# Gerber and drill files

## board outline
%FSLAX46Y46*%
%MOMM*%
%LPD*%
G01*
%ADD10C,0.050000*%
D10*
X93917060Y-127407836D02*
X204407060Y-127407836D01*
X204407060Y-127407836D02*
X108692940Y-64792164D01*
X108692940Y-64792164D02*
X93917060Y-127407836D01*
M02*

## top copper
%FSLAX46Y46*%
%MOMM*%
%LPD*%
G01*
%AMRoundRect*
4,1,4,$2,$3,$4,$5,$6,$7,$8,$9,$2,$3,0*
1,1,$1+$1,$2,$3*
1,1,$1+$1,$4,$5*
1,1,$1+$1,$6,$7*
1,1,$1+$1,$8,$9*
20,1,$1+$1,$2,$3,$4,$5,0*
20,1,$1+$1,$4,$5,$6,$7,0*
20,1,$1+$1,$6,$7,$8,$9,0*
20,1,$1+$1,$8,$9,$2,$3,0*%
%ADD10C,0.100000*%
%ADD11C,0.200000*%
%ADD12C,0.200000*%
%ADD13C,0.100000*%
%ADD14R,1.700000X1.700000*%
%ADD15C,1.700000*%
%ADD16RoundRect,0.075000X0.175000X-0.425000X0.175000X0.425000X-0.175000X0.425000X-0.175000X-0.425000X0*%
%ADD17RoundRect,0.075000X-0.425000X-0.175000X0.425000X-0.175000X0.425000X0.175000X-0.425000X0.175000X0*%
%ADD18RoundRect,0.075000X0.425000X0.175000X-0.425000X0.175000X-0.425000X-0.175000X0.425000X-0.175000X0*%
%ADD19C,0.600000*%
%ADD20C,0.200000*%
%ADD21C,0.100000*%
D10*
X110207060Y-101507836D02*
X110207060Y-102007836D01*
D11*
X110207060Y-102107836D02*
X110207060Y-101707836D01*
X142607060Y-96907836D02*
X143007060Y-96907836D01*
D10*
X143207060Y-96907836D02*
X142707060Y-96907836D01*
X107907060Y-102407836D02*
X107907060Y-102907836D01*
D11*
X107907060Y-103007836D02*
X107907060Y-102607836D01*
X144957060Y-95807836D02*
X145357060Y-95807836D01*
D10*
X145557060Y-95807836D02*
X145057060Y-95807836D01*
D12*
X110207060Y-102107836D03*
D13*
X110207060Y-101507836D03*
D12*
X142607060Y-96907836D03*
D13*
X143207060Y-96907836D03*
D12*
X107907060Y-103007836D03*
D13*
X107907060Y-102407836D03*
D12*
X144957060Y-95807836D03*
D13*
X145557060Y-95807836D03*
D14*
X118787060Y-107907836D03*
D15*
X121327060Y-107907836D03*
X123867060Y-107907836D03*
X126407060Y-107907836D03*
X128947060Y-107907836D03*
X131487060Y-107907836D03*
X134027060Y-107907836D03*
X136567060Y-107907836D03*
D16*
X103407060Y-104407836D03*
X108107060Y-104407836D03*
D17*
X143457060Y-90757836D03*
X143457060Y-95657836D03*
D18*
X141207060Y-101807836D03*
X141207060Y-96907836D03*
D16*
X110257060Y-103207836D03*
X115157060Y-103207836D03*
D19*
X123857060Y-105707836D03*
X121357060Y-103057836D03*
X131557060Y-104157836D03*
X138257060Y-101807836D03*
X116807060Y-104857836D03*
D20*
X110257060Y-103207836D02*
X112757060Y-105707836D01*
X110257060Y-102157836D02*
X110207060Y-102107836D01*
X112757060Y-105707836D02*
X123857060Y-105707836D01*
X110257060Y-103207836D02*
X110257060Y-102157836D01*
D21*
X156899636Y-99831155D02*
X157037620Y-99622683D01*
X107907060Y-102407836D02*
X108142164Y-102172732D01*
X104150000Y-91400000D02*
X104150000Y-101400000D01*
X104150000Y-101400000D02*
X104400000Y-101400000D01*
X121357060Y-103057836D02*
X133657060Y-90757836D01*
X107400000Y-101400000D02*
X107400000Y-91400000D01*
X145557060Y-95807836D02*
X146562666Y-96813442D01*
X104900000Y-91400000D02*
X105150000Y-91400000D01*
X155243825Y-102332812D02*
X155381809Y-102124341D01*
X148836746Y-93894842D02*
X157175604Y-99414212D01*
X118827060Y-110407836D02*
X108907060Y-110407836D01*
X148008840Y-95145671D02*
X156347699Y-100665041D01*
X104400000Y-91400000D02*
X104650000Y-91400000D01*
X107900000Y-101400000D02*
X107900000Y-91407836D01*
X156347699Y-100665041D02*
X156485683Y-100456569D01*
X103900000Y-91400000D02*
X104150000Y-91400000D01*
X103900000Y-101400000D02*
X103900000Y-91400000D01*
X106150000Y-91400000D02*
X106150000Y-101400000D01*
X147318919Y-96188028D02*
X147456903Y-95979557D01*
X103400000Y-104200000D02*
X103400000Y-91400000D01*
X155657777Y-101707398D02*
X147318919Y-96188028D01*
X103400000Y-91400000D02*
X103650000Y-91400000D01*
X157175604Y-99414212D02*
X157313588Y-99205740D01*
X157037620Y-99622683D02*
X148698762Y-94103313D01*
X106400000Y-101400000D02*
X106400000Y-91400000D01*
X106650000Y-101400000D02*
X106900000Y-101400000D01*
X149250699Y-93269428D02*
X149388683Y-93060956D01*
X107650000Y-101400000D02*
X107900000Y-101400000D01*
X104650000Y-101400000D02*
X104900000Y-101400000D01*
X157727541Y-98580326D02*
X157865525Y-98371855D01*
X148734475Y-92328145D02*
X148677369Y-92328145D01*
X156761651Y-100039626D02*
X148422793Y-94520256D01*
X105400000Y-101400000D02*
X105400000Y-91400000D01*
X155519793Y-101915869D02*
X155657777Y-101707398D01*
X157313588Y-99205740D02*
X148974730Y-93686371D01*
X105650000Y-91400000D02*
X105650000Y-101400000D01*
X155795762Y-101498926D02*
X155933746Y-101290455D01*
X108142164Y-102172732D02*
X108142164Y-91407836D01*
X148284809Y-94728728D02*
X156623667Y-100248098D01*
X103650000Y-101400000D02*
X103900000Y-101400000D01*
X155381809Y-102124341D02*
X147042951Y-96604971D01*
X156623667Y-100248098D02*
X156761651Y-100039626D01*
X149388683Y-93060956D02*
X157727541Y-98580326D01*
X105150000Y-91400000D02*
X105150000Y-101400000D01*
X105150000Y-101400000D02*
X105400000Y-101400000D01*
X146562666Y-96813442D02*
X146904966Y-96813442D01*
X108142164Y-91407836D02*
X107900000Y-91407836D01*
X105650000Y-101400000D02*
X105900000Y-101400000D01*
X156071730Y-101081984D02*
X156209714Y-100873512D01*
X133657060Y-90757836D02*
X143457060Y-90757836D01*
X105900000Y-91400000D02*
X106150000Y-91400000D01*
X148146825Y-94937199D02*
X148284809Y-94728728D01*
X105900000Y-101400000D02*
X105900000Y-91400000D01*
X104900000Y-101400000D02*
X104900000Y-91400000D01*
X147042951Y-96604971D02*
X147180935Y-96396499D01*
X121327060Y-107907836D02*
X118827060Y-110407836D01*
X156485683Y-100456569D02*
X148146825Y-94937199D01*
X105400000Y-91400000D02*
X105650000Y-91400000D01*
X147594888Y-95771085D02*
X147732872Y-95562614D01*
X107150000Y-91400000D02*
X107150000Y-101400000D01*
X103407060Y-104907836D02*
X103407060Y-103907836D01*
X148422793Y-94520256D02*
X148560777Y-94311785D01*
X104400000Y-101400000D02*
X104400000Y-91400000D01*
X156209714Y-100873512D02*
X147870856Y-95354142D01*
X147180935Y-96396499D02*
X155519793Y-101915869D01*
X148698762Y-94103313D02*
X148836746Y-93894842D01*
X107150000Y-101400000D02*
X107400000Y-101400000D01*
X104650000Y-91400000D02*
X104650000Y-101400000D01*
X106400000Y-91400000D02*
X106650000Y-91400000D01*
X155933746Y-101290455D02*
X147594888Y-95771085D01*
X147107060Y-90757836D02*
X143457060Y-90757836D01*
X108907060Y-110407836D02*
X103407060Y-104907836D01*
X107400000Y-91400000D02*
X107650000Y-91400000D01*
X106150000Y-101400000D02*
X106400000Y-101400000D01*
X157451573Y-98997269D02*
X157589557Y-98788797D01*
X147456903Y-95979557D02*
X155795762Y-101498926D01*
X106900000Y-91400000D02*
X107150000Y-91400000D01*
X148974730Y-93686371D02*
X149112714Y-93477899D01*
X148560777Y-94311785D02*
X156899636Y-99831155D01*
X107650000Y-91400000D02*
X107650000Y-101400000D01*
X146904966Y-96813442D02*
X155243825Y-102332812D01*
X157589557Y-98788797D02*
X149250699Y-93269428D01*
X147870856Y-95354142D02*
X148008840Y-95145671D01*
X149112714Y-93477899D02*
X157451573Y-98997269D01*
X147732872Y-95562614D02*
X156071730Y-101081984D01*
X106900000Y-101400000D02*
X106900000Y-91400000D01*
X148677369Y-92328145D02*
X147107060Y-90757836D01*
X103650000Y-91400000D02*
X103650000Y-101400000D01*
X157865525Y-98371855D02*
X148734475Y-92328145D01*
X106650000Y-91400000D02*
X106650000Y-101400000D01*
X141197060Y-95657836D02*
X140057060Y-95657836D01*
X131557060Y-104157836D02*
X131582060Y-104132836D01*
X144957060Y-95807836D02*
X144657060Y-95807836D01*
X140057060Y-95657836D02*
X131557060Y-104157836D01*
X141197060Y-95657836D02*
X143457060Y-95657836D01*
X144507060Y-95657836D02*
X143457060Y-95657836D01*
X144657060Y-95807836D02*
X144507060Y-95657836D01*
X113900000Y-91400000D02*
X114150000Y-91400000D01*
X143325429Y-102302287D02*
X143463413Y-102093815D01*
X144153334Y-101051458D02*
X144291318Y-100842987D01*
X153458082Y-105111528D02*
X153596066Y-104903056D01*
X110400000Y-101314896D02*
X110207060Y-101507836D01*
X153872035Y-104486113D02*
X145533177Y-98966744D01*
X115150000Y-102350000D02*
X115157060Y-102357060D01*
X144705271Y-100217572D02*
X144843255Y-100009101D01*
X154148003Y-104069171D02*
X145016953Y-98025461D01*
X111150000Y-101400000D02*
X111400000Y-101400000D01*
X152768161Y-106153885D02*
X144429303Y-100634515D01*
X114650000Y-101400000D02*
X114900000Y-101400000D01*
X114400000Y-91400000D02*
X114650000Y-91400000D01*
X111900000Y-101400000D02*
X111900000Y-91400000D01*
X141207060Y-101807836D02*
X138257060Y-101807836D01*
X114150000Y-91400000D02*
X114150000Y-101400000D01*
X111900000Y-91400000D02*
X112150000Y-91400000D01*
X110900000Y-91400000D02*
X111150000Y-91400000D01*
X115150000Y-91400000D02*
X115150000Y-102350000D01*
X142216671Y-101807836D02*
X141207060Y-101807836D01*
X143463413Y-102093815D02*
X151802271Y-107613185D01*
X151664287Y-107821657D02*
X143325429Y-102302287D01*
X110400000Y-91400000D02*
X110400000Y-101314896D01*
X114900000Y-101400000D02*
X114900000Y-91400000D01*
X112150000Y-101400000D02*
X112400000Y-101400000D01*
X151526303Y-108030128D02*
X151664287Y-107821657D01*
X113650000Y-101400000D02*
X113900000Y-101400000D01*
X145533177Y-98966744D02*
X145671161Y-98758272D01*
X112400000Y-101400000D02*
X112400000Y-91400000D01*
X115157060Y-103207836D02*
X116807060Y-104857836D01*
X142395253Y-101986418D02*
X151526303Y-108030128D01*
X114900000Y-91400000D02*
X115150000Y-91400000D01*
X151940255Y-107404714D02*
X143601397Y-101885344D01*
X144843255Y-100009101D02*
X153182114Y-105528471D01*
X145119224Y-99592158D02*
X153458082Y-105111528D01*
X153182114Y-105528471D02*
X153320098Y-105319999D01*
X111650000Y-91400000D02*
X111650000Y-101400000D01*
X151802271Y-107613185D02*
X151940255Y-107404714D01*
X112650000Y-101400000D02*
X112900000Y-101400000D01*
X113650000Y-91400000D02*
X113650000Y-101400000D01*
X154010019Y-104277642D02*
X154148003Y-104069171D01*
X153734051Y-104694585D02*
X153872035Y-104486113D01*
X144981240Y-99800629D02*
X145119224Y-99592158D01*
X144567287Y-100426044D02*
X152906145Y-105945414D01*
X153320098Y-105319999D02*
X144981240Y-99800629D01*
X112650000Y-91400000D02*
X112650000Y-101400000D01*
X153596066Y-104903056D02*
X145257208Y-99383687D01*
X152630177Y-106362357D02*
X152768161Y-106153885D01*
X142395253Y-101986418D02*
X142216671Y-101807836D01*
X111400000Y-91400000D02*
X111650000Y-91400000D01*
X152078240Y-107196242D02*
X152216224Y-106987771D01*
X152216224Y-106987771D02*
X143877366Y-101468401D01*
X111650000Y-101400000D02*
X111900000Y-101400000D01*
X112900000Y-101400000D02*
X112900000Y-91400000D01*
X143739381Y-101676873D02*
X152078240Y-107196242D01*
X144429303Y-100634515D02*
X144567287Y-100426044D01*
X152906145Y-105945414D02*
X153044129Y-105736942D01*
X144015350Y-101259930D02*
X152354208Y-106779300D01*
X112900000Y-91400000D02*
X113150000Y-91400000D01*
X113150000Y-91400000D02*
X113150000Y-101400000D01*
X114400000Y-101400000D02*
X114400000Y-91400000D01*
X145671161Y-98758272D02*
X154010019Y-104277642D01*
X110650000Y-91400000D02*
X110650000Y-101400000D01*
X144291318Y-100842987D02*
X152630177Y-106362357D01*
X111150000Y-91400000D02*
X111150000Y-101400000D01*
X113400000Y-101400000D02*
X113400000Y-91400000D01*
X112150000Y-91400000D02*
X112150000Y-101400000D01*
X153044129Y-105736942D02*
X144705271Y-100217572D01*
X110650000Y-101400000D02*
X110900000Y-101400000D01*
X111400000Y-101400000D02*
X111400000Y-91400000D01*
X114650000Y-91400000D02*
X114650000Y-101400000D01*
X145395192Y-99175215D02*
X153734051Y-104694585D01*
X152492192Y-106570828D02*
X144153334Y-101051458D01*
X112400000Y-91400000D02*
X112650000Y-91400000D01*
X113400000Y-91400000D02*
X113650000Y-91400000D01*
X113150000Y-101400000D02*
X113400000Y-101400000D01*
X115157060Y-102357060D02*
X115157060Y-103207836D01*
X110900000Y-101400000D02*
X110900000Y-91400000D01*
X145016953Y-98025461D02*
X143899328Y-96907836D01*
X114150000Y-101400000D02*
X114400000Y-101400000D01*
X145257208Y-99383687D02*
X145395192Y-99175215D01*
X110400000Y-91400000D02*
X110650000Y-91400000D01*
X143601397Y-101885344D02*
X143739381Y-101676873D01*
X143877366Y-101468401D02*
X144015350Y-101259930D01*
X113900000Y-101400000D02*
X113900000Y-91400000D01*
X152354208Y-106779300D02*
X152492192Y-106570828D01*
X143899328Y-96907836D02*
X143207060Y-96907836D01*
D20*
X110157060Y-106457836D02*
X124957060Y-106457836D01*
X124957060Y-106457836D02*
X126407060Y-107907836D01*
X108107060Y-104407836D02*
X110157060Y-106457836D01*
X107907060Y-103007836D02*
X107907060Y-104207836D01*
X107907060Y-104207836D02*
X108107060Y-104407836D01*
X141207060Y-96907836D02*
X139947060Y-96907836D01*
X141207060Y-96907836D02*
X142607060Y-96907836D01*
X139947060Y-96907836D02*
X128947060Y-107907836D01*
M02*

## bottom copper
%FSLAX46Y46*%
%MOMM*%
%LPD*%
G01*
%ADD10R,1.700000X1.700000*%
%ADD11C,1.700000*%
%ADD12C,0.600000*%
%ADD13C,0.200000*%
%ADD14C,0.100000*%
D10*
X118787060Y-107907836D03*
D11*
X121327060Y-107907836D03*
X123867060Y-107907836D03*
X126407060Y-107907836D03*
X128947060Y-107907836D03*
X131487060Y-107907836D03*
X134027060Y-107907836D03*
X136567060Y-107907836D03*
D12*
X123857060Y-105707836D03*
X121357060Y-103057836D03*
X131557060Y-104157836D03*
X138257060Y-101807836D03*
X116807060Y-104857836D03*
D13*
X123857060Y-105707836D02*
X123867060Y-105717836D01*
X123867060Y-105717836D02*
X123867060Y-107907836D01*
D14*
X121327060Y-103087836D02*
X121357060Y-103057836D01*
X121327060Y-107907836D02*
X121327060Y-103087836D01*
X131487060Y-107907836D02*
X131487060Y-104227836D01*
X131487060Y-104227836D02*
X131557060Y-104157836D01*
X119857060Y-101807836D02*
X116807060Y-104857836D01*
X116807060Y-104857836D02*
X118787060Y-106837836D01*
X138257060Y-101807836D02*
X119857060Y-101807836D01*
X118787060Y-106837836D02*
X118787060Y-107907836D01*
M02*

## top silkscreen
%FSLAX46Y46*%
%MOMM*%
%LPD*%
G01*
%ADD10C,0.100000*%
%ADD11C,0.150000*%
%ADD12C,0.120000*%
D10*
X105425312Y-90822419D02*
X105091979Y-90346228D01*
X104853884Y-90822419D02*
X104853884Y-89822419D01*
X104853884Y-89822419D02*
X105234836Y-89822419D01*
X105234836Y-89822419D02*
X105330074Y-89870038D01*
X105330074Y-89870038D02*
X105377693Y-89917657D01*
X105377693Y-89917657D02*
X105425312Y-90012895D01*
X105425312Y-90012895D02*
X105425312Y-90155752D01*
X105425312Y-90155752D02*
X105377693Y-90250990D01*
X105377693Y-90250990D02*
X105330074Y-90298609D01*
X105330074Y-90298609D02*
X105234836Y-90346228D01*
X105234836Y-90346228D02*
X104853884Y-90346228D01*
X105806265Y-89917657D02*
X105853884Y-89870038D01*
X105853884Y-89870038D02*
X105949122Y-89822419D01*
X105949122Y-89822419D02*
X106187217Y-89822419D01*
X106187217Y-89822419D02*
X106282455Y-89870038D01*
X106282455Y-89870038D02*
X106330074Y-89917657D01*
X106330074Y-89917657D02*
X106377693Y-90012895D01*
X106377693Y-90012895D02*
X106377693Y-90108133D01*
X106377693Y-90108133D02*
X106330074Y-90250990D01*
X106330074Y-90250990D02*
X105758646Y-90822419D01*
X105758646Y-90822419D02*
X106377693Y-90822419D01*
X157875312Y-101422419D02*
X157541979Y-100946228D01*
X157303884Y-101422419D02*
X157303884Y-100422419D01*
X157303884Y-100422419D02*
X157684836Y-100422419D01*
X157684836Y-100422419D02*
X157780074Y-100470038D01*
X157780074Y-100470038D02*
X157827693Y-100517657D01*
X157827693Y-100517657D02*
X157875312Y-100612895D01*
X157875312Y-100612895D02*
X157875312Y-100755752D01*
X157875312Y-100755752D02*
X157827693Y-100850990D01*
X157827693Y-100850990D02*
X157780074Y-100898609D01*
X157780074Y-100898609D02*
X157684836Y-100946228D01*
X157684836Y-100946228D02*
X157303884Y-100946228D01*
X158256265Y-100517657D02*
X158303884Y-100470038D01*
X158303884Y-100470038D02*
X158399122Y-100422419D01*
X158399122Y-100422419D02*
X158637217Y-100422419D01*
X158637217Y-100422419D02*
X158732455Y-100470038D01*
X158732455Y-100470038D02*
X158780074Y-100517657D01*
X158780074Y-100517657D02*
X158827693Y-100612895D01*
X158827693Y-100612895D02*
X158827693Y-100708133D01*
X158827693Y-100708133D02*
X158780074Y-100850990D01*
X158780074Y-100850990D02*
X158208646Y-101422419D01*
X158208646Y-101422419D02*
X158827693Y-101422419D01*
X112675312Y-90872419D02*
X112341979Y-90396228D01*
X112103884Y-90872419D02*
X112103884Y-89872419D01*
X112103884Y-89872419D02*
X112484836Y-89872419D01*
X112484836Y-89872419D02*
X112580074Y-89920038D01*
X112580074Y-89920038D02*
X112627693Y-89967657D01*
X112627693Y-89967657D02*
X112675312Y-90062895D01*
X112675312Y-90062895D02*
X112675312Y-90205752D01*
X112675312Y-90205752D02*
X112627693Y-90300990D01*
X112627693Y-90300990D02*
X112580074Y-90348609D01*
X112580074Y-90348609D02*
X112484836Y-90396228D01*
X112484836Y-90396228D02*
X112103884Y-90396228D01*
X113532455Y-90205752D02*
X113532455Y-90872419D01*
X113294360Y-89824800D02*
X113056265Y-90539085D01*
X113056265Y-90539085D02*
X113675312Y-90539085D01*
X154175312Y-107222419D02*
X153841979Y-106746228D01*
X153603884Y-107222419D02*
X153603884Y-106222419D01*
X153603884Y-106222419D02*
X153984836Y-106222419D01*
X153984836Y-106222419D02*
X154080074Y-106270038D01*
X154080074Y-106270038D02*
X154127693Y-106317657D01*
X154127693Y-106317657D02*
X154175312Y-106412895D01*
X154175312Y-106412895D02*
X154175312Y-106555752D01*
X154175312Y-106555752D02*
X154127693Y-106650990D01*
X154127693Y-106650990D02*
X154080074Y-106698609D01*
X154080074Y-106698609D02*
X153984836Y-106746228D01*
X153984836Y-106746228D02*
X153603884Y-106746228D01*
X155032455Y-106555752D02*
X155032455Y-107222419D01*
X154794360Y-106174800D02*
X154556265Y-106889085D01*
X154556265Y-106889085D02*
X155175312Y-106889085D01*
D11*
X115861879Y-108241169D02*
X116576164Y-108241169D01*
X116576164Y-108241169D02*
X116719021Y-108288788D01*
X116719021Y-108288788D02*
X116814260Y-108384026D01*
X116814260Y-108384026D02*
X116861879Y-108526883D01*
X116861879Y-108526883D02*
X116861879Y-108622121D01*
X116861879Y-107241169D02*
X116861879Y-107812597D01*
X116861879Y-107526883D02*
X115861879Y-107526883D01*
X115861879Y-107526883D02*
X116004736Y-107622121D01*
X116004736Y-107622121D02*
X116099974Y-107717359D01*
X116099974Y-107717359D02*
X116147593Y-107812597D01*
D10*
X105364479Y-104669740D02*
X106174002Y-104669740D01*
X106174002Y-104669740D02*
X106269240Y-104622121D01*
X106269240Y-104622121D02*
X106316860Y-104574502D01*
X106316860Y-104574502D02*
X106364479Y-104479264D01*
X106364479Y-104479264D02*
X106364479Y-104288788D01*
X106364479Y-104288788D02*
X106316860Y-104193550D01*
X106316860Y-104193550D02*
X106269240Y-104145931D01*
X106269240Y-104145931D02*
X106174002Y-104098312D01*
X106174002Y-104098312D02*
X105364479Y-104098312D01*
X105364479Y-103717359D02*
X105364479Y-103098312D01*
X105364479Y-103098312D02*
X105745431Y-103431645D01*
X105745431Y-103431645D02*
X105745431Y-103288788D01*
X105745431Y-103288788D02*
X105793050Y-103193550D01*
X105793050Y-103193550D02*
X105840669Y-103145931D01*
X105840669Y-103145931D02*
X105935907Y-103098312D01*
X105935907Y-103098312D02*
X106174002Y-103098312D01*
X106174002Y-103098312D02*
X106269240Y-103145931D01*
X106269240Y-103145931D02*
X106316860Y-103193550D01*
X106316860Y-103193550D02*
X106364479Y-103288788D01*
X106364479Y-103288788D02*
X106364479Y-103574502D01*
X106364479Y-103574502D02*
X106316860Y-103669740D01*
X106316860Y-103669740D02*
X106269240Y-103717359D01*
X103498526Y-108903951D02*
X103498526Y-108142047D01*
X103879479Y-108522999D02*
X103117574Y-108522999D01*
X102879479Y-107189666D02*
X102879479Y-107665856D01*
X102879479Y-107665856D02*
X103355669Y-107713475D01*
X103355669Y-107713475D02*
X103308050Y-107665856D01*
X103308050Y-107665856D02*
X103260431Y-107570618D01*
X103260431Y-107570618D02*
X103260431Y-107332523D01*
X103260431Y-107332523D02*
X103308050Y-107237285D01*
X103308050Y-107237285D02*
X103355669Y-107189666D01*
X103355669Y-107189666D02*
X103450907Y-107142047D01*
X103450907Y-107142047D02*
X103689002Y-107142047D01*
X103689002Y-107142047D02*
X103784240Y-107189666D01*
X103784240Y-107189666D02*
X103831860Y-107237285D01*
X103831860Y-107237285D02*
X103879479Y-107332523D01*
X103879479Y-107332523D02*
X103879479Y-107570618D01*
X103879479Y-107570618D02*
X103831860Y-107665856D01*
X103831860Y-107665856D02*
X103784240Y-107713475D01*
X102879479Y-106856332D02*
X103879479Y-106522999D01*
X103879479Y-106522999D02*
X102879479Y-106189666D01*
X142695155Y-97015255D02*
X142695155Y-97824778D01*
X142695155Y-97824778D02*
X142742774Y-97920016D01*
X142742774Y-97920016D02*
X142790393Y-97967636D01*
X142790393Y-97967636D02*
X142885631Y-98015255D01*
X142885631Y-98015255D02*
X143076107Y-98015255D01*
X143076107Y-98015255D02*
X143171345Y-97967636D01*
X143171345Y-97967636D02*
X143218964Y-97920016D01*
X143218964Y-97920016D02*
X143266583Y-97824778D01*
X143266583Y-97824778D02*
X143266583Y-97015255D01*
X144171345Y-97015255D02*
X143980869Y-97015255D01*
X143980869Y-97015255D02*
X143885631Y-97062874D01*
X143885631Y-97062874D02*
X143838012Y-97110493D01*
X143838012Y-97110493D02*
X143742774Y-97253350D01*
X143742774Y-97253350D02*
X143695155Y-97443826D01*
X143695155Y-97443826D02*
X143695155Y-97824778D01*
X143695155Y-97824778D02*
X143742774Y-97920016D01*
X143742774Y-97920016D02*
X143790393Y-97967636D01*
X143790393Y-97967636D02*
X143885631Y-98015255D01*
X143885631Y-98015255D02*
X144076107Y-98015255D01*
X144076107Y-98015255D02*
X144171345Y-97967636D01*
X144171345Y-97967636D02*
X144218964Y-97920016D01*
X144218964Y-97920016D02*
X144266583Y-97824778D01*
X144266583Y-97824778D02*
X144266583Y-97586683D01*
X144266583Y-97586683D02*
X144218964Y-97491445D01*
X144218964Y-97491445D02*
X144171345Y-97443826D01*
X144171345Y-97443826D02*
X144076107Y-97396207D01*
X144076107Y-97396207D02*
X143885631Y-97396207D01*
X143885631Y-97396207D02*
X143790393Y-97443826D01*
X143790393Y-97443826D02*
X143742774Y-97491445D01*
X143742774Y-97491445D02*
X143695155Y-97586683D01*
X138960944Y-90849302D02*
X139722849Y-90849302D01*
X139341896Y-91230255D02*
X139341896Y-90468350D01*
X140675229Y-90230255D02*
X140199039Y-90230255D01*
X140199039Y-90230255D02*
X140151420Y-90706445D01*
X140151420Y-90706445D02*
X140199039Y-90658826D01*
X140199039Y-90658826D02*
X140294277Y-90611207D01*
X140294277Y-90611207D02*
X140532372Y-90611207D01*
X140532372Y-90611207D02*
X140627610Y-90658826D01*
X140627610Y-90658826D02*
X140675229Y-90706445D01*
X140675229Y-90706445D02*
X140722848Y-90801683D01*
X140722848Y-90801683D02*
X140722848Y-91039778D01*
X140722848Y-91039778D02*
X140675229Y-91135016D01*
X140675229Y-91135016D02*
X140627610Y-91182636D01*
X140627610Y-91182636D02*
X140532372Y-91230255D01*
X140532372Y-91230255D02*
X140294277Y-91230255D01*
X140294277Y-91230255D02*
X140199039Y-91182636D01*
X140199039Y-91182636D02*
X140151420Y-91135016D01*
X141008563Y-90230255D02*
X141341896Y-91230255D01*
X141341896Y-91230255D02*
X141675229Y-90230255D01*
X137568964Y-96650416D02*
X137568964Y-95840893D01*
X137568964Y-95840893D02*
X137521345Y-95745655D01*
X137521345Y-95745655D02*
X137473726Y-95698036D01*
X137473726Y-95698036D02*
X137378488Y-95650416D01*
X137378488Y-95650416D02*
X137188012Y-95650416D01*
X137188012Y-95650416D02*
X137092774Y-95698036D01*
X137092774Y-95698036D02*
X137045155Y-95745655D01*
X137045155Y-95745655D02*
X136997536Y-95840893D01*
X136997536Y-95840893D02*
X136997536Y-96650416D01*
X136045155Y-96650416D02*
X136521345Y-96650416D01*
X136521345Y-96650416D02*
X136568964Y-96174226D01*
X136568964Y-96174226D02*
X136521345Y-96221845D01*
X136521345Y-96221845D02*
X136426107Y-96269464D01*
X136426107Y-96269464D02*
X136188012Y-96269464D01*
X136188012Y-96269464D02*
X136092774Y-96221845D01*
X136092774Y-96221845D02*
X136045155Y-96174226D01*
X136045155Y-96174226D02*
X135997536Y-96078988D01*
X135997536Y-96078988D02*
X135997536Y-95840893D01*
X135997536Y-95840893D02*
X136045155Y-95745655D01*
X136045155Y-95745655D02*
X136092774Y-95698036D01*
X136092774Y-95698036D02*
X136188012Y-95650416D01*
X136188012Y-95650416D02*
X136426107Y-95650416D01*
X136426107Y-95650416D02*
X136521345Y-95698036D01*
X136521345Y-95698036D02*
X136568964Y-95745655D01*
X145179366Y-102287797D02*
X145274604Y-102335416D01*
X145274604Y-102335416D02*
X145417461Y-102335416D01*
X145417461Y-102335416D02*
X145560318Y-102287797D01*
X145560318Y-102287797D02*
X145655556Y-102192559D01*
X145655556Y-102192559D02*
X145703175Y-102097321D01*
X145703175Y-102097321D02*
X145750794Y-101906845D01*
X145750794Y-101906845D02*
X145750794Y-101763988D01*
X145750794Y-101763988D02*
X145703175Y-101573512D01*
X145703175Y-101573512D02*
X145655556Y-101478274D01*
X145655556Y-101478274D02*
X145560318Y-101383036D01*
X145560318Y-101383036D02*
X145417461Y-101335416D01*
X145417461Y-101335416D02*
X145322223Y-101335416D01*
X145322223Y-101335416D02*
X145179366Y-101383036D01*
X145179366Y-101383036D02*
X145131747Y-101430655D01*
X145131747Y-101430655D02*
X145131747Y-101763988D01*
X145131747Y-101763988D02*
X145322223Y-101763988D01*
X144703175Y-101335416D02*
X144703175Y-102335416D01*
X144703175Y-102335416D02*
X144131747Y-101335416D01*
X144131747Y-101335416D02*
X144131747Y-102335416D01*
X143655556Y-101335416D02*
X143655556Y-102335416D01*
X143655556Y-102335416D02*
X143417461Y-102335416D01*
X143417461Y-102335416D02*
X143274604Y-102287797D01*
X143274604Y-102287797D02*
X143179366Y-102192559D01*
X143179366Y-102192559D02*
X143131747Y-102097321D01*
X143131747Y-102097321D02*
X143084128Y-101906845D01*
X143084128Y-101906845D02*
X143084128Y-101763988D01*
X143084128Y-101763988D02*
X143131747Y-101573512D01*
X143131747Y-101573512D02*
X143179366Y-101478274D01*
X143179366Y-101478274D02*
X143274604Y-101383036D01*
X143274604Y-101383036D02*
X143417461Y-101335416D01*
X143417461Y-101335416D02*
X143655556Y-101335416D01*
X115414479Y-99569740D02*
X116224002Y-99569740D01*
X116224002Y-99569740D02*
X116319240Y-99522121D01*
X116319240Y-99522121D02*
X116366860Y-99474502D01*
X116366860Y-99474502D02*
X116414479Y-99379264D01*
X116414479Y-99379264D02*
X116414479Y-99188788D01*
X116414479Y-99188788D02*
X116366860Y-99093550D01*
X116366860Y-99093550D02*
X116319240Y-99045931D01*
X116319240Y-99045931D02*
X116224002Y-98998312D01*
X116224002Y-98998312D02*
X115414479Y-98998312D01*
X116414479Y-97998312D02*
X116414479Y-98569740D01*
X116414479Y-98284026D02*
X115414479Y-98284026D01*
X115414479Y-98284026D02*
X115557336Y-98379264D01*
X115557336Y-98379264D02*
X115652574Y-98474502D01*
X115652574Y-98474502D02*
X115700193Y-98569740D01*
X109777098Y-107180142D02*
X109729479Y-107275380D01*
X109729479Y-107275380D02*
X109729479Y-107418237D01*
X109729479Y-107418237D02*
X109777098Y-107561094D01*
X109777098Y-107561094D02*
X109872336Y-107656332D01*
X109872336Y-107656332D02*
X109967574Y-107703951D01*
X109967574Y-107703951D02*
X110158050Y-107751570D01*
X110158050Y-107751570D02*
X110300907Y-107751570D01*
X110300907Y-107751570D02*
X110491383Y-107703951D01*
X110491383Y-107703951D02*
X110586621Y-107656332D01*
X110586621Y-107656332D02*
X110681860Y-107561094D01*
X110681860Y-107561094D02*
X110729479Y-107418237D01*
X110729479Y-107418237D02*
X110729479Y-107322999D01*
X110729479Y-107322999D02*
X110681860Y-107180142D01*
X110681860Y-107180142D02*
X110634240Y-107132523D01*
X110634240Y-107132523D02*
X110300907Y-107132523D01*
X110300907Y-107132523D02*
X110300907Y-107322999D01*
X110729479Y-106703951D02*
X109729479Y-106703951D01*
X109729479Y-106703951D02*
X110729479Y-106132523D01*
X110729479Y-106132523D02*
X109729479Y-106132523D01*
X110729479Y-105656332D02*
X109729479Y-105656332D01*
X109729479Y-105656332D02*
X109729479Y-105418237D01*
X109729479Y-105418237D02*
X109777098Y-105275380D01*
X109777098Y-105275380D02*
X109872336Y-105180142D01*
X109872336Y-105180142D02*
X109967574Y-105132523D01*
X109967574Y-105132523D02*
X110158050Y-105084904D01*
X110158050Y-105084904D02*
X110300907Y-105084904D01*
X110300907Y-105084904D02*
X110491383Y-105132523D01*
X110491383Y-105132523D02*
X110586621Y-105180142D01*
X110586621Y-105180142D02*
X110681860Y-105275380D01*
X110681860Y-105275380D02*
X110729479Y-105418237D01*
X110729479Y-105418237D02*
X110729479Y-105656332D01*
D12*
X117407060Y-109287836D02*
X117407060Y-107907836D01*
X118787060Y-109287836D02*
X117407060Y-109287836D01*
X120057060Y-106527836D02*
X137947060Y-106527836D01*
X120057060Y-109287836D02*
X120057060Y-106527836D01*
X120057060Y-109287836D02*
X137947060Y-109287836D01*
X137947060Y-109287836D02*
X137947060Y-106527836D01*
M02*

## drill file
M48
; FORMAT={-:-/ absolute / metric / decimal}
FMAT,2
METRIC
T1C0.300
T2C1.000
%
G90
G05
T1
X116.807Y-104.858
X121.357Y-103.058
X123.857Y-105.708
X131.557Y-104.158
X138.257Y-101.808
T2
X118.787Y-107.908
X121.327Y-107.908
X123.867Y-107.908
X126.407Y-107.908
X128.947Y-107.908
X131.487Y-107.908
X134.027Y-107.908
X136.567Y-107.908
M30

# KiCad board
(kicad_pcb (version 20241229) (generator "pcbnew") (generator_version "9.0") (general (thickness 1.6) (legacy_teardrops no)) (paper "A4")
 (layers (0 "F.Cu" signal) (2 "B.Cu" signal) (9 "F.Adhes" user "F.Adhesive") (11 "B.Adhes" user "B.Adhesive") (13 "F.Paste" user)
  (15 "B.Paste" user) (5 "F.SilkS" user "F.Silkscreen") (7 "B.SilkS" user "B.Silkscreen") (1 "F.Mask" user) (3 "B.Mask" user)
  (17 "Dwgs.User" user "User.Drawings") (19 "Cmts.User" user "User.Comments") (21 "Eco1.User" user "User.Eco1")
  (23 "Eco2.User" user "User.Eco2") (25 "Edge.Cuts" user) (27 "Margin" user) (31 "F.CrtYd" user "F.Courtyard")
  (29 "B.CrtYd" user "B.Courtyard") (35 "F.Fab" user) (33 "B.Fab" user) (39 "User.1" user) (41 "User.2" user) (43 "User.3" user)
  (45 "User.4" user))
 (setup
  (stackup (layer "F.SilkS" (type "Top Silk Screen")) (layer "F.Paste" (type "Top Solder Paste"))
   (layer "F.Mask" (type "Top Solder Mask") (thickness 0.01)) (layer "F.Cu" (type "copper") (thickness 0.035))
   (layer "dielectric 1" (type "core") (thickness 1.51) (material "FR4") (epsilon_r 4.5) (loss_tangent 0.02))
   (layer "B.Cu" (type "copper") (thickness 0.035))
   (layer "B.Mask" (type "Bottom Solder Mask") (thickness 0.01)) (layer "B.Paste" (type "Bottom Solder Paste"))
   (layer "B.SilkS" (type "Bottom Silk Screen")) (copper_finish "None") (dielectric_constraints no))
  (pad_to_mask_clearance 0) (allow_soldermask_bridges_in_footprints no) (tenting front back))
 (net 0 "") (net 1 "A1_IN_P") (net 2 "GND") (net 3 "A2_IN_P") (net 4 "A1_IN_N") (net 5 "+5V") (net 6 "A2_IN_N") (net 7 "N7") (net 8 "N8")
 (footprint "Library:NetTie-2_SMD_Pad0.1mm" (layer "F.Cu") (at 110.20706 102.007836 90)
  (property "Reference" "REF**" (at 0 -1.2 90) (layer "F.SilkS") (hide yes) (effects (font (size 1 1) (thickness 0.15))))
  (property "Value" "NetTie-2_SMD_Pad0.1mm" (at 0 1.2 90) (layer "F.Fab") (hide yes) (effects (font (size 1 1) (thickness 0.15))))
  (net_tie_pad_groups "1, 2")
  (fp_line (start 0.5 0) (end 0 0) (stroke (width 0.1) (type solid)) (layer "F.Cu"))
  (fp_line (start -0.1 0) (end 0.3 0) (stroke (width 0.2) (type solid)) (layer "F.Cu"))
  (pad "1" smd circle (at -0.1 0 90) (size 0.2 0.2) (layers "F.Cu") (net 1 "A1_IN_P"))
  (pad "2" smd circle (at 0.5 0 90) (size 0.1 0.1) (layers "F.Cu") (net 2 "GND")))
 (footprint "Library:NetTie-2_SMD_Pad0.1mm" (layer "F.Cu") (at 142.70706 96.907836)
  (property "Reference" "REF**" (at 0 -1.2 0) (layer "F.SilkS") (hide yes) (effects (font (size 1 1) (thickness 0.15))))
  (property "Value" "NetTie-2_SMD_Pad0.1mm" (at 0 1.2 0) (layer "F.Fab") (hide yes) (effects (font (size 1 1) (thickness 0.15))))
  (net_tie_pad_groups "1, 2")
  (fp_line (start -0.1 0) (end 0.3 0) (stroke (width 0.2) (type solid)) (layer "F.Cu"))
  (fp_line (start 0.5 0) (end 0 0) (stroke (width 0.1) (type solid)) (layer "F.Cu"))
  (pad "1" smd circle (at -0.1 0) (size 0.2 0.2) (layers "F.Cu") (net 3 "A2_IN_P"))
  (pad "2" smd circle (at 0.5 0) (size 0.1 0.1) (layers "F.Cu") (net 2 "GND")))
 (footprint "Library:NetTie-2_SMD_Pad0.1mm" (layer "F.Cu") (at 107.90706 102.907836 90)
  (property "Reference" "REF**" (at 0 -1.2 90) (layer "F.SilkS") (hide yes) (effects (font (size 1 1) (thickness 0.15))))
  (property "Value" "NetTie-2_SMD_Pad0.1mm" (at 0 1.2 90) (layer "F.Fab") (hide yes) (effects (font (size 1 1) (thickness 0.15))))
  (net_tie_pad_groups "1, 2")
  (fp_line (start 0.5 0) (end 0 0) (stroke (width 0.1) (type solid)) (layer "F.Cu"))
  (fp_line (start -0.1 0) (end 0.3 0) (stroke (width 0.2) (type solid)) (layer "F.Cu"))
  (pad "1" smd circle (at -0.1 0 90) (size 0.2 0.2) (layers "F.Cu") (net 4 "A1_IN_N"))
  (pad "2" smd circle (at 0.5 0 90) (size 0.1 0.1) (layers "F.Cu") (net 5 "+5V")))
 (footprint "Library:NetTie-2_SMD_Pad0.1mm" (layer "F.Cu") (at 145.05706 95.807836)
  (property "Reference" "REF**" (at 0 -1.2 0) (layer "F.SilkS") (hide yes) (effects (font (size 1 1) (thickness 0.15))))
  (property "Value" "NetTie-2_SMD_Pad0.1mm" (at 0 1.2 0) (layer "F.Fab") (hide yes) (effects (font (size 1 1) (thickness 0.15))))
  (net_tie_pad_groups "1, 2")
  (fp_line (start -0.1 0) (end 0.3 0) (stroke (width 0.2) (type solid)) (layer "F.Cu"))
  (fp_line (start 0.5 0) (end 0 0) (stroke (width 0.1) (type solid)) (layer "F.Cu"))
  (pad "1" smd circle (at -0.1 0) (size 0.2 0.2) (layers "F.Cu") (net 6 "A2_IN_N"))
  (pad "2" smd circle (at 0.5 0) (size 0.1 0.1) (layers "F.Cu") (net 5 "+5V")))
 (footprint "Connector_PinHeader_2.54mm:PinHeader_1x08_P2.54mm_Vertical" (layer "F.Cu") (at 118.78706 107.907836 90)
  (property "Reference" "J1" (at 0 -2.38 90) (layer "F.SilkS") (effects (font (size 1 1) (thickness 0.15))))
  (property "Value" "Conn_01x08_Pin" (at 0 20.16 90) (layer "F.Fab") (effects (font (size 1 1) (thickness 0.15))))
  (fp_line (start -1.38 -1.38) (end 0 -1.38) (stroke (width 0.12) (type solid)) (layer "F.SilkS"))
  (fp_line (start -1.38 0) (end -1.38 -1.38) (stroke (width 0.12) (type solid)) (layer "F.SilkS"))
  (fp_line (start 1.38 1.27) (end 1.38 19.16) (stroke (width 0.12) (type solid)) (layer "F.SilkS"))
  (fp_line (start -1.38 1.27) (end 1.38 1.27) (stroke (width 0.12) (type solid)) (layer "F.SilkS"))
  (fp_line (start -1.38 1.27) (end -1.38 19.16) (stroke (width 0.12) (type solid)) (layer "F.SilkS"))
  (fp_line (start -1.38 19.16) (end 1.38 19.16) (stroke (width 0.12) (type solid)) (layer "F.SilkS"))
  (pad "1" thru_hole rect (at 0 0 90) (size 1.7 1.7) (drill 1) (layers "*.Cu" "*.Mask") (remove_unused_layers no) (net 2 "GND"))
  (pad "2" thru_hole circle (at 0 2.54 90) (size 1.7 1.7) (drill 1) (layers "*.Cu" "*.Mask") (remove_unused_layers no) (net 5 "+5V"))
  (pad "3" thru_hole circle (at 0 5.08 90) (size 1.7 1.7) (drill 1) (layers "*.Cu" "*.Mask") (remove_unused_layers no) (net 1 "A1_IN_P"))
  (pad "4" thru_hole circle (at 0 7.62 90) (size 1.7 1.7) (drill 1) (layers "*.Cu" "*.Mask") (remove_unused_layers no) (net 4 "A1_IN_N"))
  (pad "5" thru_hole circle (at 0 10.16 90) (size 1.7 1.7) (drill 1) (layers "*.Cu" "*.Mask") (remove_unused_layers no) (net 3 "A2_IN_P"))
  (pad "6" thru_hole circle (at 0 12.7 90) (size 1.7 1.7) (drill 1) (layers "*.Cu" "*.Mask") (remove_unused_layers no) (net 6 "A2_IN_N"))
  (pad "7" thru_hole circle (at 0 15.24 90) (size 1.7 1.7) (drill 1) (layers "*.Cu" "*.Mask") (remove_unused_layers no) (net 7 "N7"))
  (pad "8" thru_hole circle (at 0 17.78 90) (size 1.7 1.7) (drill 1) (layers "*.Cu" "*.Mask") (remove_unused_layers no) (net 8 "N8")))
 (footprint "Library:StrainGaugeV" (layer "F.Cu") (at 110.70706 104.407836 90)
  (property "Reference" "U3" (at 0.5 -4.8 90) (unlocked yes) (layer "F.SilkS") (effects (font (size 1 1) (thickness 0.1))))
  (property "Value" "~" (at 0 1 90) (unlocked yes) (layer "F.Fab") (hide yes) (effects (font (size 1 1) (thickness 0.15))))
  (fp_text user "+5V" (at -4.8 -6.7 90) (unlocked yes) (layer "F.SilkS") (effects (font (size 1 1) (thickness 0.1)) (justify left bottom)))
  (pad "1" smd roundrect (at 0 -7.3 90) (size 1 0.5) (layers "F.Cu" "F.Mask" "F.Paste") (roundrect_rratio 0.15) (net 5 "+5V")
   (thermal_bridge_angle 45))
  (pad "2" smd roundrect (at 0 -2.6 90) (size 1 0.5) (layers "F.Cu" "F.Mask" "F.Paste") (roundrect_rratio 0.15) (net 4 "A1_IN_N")
   (thermal_bridge_angle 45)))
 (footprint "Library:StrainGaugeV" (layer "F.Cu") (at 143.45706 98.057836)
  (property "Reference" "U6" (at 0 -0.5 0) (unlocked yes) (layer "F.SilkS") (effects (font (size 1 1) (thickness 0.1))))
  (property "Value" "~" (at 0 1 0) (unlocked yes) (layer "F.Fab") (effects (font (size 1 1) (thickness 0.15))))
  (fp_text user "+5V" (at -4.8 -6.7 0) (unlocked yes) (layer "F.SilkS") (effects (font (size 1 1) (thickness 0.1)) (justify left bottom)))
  (pad "1" smd roundrect (at 0 -7.3) (size 1 0.5) (layers "F.Cu" "F.Mask" "F.Paste") (roundrect_rratio 0.15) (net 5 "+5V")
   (thermal_bridge_angle 45))
  (pad "2" smd roundrect (at 0 -2.4) (size 1 0.5) (layers "F.Cu" "F.Mask" "F.Paste") (roundrect_rratio 0.15) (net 6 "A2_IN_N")
   (thermal_bridge_angle 45)))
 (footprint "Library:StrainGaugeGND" (layer "F.Cu") (at 141.20706 96.907836 180)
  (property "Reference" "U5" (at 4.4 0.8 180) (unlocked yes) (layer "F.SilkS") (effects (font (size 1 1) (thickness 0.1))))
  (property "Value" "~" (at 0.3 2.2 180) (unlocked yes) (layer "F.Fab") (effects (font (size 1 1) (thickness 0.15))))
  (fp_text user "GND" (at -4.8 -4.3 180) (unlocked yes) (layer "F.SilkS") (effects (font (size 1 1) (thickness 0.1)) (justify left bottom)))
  (pad "1" smd roundrect (at 0 -4.9 180) (size 1 0.5) (layers "F.Cu" "F.Mask" "F.Paste") (roundrect_rratio 0.15) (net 2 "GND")
   (thermal_bridge_angle 45))
  (pad "2" smd roundrect (at 0 0 180) (size 1 0.5) (layers "F.Cu" "F.Mask" "F.Paste") (roundrect_rratio 0.15) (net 3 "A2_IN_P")
   (thermal_bridge_angle 45)))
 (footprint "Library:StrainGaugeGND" (layer "F.Cu") (at 115.15706 103.207836 90)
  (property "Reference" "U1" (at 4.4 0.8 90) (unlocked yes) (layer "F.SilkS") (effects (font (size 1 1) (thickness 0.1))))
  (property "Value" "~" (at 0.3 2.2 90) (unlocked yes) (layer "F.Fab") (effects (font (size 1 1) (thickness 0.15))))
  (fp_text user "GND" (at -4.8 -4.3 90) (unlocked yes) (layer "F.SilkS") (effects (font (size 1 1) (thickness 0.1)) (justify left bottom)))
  (pad "1" smd roundrect (at 0 -4.9 90) (size 1 0.5) (layers "F.Cu" "F.Mask" "F.Paste") (roundrect_rratio 0.15) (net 1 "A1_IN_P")
   (thermal_bridge_angle 45))
  (pad "2" smd roundrect (at 0 0 90) (size 1 0.5) (layers "F.Cu" "F.Mask" "F.Paste") (roundrect_rratio 0.15) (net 2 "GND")
   (thermal_bridge_angle 45)))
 (gr_line (start 93.91706 127.407836) (end 204.40706 127.407836) (stroke (width 0.05) (type default)) (layer "Edge.Cuts"))
 (gr_line (start 204.40706 127.407836) (end 108.69294 64.792164) (stroke (width 0.05) (type solid)) (layer "Edge.Cuts"))
 (gr_line (start 108.69294 64.792164) (end 93.91706 127.407836) (stroke (width 0.05) (type solid)) (layer "Edge.Cuts"))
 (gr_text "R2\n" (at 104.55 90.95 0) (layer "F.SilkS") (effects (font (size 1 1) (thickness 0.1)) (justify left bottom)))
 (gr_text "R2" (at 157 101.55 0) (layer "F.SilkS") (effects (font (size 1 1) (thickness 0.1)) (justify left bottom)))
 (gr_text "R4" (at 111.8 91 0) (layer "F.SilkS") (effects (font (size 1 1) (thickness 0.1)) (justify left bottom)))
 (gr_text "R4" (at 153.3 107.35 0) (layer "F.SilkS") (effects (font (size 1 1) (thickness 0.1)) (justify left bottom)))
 (segment (start 110.25706 103.207836) (end 112.75706 105.707836) (width 0.2) (layer "F.Cu") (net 1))
 (segment (start 110.25706 102.157836) (end 110.20706 102.107836) (width 0.2) (layer "F.Cu") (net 1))
 (segment (start 112.75706 105.707836) (end 123.85706 105.707836) (width 0.2) (layer "F.Cu") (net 1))
 (segment (start 110.25706 103.207836) (end 110.25706 102.157836) (width 0.2) (layer "F.Cu") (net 1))
 (via (at 123.85706 105.707836) (size 0.6) (drill 0.3) (layers "F.Cu" "B.Cu") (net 1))
 (segment (start 123.85706 105.707836) (end 123.86706 105.717836) (width 0.2) (layer "B.Cu") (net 1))
 (segment (start 123.86706 105.717836) (end 123.86706 107.907836) (width 0.2) (layer "B.Cu") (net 1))
 (segment (start 156.899636 99.831155) (end 157.03762 99.622683) (width 0.1) (layer "F.Cu") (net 5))
 (segment (start 107.90706 102.407836) (end 108.142164 102.172732) (width 0.1) (layer "F.Cu") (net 5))
 (segment (start 104.15 91.4) (end 104.15 101.4) (width 0.1) (layer "F.Cu") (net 5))
 (segment (start 104.15 101.4) (end 104.4 101.4) (width 0.1) (layer "F.Cu") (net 5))
 (segment (start 121.35706 103.057836) (end 133.65706 90.757836) (width 0.1) (layer "F.Cu") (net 5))
 (segment (start 107.4 101.4) (end 107.4 91.4) (width 0.1) (layer "F.Cu") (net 5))
 (segment (start 145.55706 95.807836) (end 146.562666 96.813442) (width 0.1) (layer "F.Cu") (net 5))
 (segment (start 104.9 91.4) (end 105.15 91.4) (width 0.1) (layer "F.Cu") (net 5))
 (segment (start 155.243825 102.332812) (end 155.381809 102.124341) (width 0.1) (layer "F.Cu") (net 5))
 (segment (start 148.836746 93.894842) (end 157.175604 99.414212) (width 0.1) (layer "F.Cu") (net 5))
 (segment (start 118.82706 110.407836) (end 108.90706 110.407836) (width 0.1) (layer "F.Cu") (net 5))
 (segment (start 148.00884 95.145671) (end 156.347699 100.665041) (width 0.1) (layer "F.Cu") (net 5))
 (segment (start 104.4 91.4) (end 104.65 91.4) (width 0.1) (layer "F.Cu") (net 5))
 (segment (start 107.9 101.4) (end 107.9 91.407836) (width 0.1) (layer "F.Cu") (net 5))
 (segment (start 156.347699 100.665041) (end 156.485683 100.456569) (width 0.1) (layer "F.Cu") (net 5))
 (segment (start 103.9 91.4) (end 104.15 91.4) (width 0.1) (layer "F.Cu") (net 5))
 (segment (start 103.9 101.4) (end 103.9 91.4) (width 0.1) (layer "F.Cu") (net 5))
 (segment (start 106.15 91.4) (end 106.15 101.4) (width 0.1) (layer "F.Cu") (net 5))
 (segment (start 147.318919 96.188028) (end 147.456903 95.979557) (width 0.1) (layer "F.Cu") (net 5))
 (segment (start 103.4 104.2) (end 103.4 91.4) (width 0.1) (layer "F.Cu") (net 5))
 (segment (start 155.657777 101.707398) (end 147.318919 96.188028) (width 0.1) (layer "F.Cu") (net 5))
 (segment (start 103.4 91.4) (end 103.65 91.4) (width 0.1) (layer "F.Cu") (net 5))
 (segment (start 157.175604 99.414212) (end 157.313588 99.20574) (width 0.1) (layer "F.Cu") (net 5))
 (segment (start 157.03762 99.622683) (end 148.698762 94.103313) (width 0.1) (layer "F.Cu") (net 5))
 (segment (start 106.4 101.4) (end 106.4 91.4) (width 0.1) (layer "F.Cu") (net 5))
 (segment (start 106.65 101.4) (end 106.9 101.4) (width 0.1) (layer "F.Cu") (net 5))
 (segment (start 149.250699 93.269428) (end 149.388683 93.060956) (width 0.1) (layer "F.Cu") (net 5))
 (segment (start 107.65 101.4) (end 107.9 101.4) (width 0.1) (layer "F.Cu") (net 5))
 (segment (start 104.65 101.4) (end 104.9 101.4) (width 0.1) (layer "F.Cu") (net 5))
 (segment (start 157.727541 98.580326) (end 157.865525 98.371855) (width 0.1) (layer "F.Cu") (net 5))
 (segment (start 148.734475 92.328145) (end 148.677369 92.328145) (width 0.1) (layer "F.Cu") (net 5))
 (segment (start 156.761651 100.039626) (end 148.422793 94.520256) (width 0.1) (layer "F.Cu") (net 5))
 (segment (start 105.4 101.4) (end 105.4 91.4) (width 0.1) (layer "F.Cu") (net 5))
 (segment (start 155.519793 101.915869) (end 155.657777 101.707398) (width 0.1) (layer "F.Cu") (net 5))
 (segment (start 157.313588 99.20574) (end 148.97473 93.686371) (width 0.1) (layer "F.Cu") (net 5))
 (segment (start 105.65 91.4) (end 105.65 101.4) (width 0.1) (layer "F.Cu") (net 5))
 (segment (start 155.795762 101.498926) (end 155.933746 101.290455) (width 0.1) (layer "F.Cu") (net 5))
 (segment (start 108.142164 102.172732) (end 108.142164 91.407836) (width 0.1) (layer "F.Cu") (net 5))
 (segment (start 148.284809 94.728728) (end 156.623667 100.248098) (width 0.1) (layer "F.Cu") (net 5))
 (segment (start 103.65 101.4) (end 103.9 101.4) (width 0.1) (layer "F.Cu") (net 5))
 (segment (start 155.381809 102.124341) (end 147.042951 96.604971) (width 0.1) (layer "F.Cu") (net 5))
 (segment (start 156.623667 100.248098) (end 156.761651 100.039626) (width 0.1) (layer "F.Cu") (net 5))
 (segment (start 149.388683 93.060956) (end 157.727541 98.580326) (width 0.1) (layer "F.Cu") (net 5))
 (segment (start 105.15 91.4) (end 105.15 101.4) (width 0.1) (layer "F.Cu") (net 5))
 (segment (start 105.15 101.4) (end 105.4 101.4) (width 0.1) (layer "F.Cu") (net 5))
 (segment (start 146.562666 96.813442) (end 146.904966 96.813442) (width 0.1) (layer "F.Cu") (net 5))
 (segment (start 108.142164 91.407836) (end 107.9 91.407836) (width 0.1) (layer "F.Cu") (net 5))
 (segment (start 105.65 101.4) (end 105.9 101.4) (width 0.1) (layer "F.Cu") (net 5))
 (segment (start 156.07173 101.081984) (end 156.209714 100.873512) (width 0.1) (layer "F.Cu") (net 5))
 (segment (start 133.65706 90.757836) (end 143.45706 90.757836) (width 0.1) (layer "F.Cu") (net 5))
 (segment (start 105.9 91.4) (end 106.15 91.4) (width 0.1) (layer "F.Cu") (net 5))
 (segment (start 148.146825 94.937199) (end 148.284809 94.728728) (width 0.1) (layer "F.Cu") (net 5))
 (segment (start 105.9 101.4) (end 105.9 91.4) (width 0.1) (layer "F.Cu") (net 5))
 (segment (start 104.9 101.4) (end 104.9 91.4) (width 0.1) (layer "F.Cu") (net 5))
 (segment (start 147.042951 96.604971) (end 147.180935 96.396499) (width 0.1) (layer "F.Cu") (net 5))
 (segment (start 121.32706 107.907836) (end 118.82706 110.407836) (width 0.1) (layer "F.Cu") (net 5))
 (segment (start 156.485683 100.456569) (end 148.146825 94.937199) (width 0.1) (layer "F.Cu") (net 5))
 (segment (start 105.4 91.4) (end 105.65 91.4) (width 0.1) (layer "F.Cu") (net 5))
 (segment (start 147.594888 95.771085) (end 147.732872 95.562614) (width 0.1) (layer "F.Cu") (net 5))
 (segment (start 107.15 91.4) (end 107.15 101.4) (width 0.1) (layer "F.Cu") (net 5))
 (segment (start 103.40706 104.907836) (end 103.40706 103.907836) (width 0.1) (layer "F.Cu") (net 5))
 (segment (start 148.422793 94.520256) (end 148.560777 94.311785) (width 0.1) (layer "F.Cu") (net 5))
 (segment (start 104.4 101.4) (end 104.4 91.4) (width 0.1) (layer "F.Cu") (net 5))
 (segment (start 156.209714 100.873512) (end 147.870856 95.354142) (width 0.1) (layer "F.Cu") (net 5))
 (segment (start 147.180935 96.396499) (end 155.519793 101.915869) (width 0.1) (layer "F.Cu") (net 5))
 (segment (start 148.698762 94.103313) (end 148.836746 93.894842) (width 0.1) (layer "F.Cu") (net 5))
 (segment (start 107.15 101.4) (end 107.4 101.4) (width 0.1) (layer "F.Cu") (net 5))
 (segment (start 104.65 91.4) (end 104.65 101.4) (width 0.1) (layer "F.Cu") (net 5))
 (segment (start 106.4 91.4) (end 106.65 91.4) (width 0.1) (layer "F.Cu") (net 5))
 (segment (start 155.933746 101.290455) (end 147.594888 95.771085) (width 0.1) (layer "F.Cu") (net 5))
 (segment (start 147.10706 90.757836) (end 143.45706 90.757836) (width 0.1) (layer "F.Cu") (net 5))
 (segment (start 108.90706 110.407836) (end 103.40706 104.907836) (width 0.1) (layer "F.Cu") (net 5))
 (segment (start 107.4 91.4) (end 107.65 91.4) (width 0.1) (layer "F.Cu") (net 5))
 (segment (start 106.15 101.4) (end 106.4 101.4) (width 0.1) (layer "F.Cu") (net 5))
 (segment (start 157.451573 98.997269) (end 157.589557 98.788797) (width 0.1) (layer "F.Cu") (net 5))
 (segment (start 147.456903 95.979557) (end 155.795762 101.498926) (width 0.1) (layer "F.Cu") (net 5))
 (segment (start 106.9 91.4) (end 107.15 91.4) (width 0.1) (layer "F.Cu") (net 5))
 (segment (start 148.97473 93.686371) (end 149.112714 93.477899) (width 0.1) (layer "F.Cu") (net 5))
 (segment (start 148.560777 94.311785) (end 156.899636 99.831155) (width 0.1) (layer "F.Cu") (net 5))
 (segment (start 107.65 91.4) (end 107.65 101.4) (width 0.1) (layer "F.Cu") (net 5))
 (segment (start 146.904966 96.813442) (end 155.243825 102.332812) (width 0.1) (layer "F.Cu") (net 5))
 (segment (start 157.589557 98.788797) (end 149.250699 93.269428) (width 0.1) (layer "F.Cu") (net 5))
 (segment (start 147.870856 95.354142) (end 148.00884 95.145671) (width 0.1) (layer "F.Cu") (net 5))
 (segment (start 149.112714 93.477899) (end 157.451573 98.997269) (width 0.1) (layer "F.Cu") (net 5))
 (segment (start 147.732872 95.562614) (end 156.07173 101.081984) (width 0.1) (layer "F.Cu") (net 5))
 (segment (start 106.9 101.4) (end 106.9 91.4) (width 0.1) (layer "F.Cu") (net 5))
 (segment (start 148.677369 92.328145) (end 147.10706 90.757836) (width 0.1) (layer "F.Cu") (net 5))
 (segment (start 103.65 91.4) (end 103.65 101.4) (width 0.1) (layer "F.Cu") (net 5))
 (segment (start 157.865525 98.371855) (end 148.734475 92.328145) (width 0.1) (layer "F.Cu") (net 5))
 (segment (start 106.65 91.4) (end 106.65 101.4) (width 0.1) (layer "F.Cu") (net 5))
 (via (at 121.35706 103.057836) (size 0.6) (drill 0.3) (layers "F.Cu" "B.Cu") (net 5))
 (segment (start 121.32706 103.087836) (end 121.35706 103.057836) (width 0.1) (layer "B.Cu") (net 5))
 (segment (start 121.32706 107.907836) (end 121.32706 103.087836) (width 0.1) (layer "B.Cu") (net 5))
 (segment (start 141.19706 95.657836) (end 140.05706 95.657836) (width 0.1) (layer "F.Cu") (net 6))
 (segment (start 131.55706 104.157836) (end 131.58206 104.132836) (width 0.1) (layer "F.Cu") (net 6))
 (segment (start 144.95706 95.807836) (end 144.65706 95.807836) (width 0.1) (layer "F.Cu") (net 6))
 (segment (start 140.05706 95.657836) (end 131.55706 104.157836) (width 0.1) (layer "F.Cu") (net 6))
 (segment (start 141.19706 95.657836) (end 143.45706 95.657836) (width 0.1) (layer "F.Cu") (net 6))
 (segment (start 144.50706 95.657836) (end 143.45706 95.657836) (width 0.1) (layer "F.Cu") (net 6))
 (segment (start 144.65706 95.807836) (end 144.50706 95.657836) (width 0.1) (layer "F.Cu") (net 6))
 (via (at 131.55706 104.157836) (size 0.6) (drill 0.3) (layers "F.Cu" "B.Cu") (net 6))
 (segment (start 131.48706 107.907836) (end 131.48706 104.227836) (width 0.1) (layer "B.Cu") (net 6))
 (segment (start 131.48706 104.227836) (end 131.55706 104.157836) (width 0.1) (layer "B.Cu") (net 6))
 (segment (start 113.9 91.4) (end 114.15 91.4) (width 0.1) (layer "F.Cu") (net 2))
 (segment (start 143.325429 102.302287) (end 143.463413 102.093815) (width 0.1) (layer "F.Cu") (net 2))
 (segment (start 144.153334 101.051458) (end 144.291318 100.842987) (width 0.1) (layer "F.Cu") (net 2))
 (segment (start 153.458082 105.111528) (end 153.596066 104.903056) (width 0.1) (layer "F.Cu") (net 2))
 (segment (start 110.4 101.314896) (end 110.20706 101.507836) (width 0.1) (layer "F.Cu") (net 2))
 (segment (start 153.872035 104.486113) (end 145.533177 98.966744) (width 0.1) (layer "F.Cu") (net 2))
 (segment (start 115.15 102.35) (end 115.15706 102.35706) (width 0.1) (layer "F.Cu") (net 2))
 (segment (start 144.705271 100.217572) (end 144.843255 100.009101) (width 0.1) (layer "F.Cu") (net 2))
 (segment (start 154.148003 104.069171) (end 145.016953 98.025461) (width 0.1) (layer "F.Cu") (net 2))
 (segment (start 111.15 101.4) (end 111.4 101.4) (width 0.1) (layer "F.Cu") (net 2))
 (segment (start 152.768161 106.153885) (end 144.429303 100.634515) (width 0.1) (layer "F.Cu") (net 2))
 (segment (start 114.65 101.4) (end 114.9 101.4) (width 0.1) (layer "F.Cu") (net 2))
 (segment (start 114.4 91.4) (end 114.65 91.4) (width 0.1) (layer "F.Cu") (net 2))
 (segment (start 111.9 101.4) (end 111.9 91.4) (width 0.1) (layer "F.Cu") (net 2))
 (segment (start 141.20706 101.807836) (end 138.25706 101.807836) (width 0.1) (layer "F.Cu") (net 2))
 (segment (start 114.15 91.4) (end 114.15 101.4) (width 0.1) (layer "F.Cu") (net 2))
 (segment (start 111.9 91.4) (end 112.15 91.4) (width 0.1) (layer "F.Cu") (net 2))
 (segment (start 110.9 91.4) (end 111.15 91.4) (width 0.1) (layer "F.Cu") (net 2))
 (segment (start 115.15 91.4) (end 115.15 102.35) (width 0.1) (layer "F.Cu") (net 2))
 (segment (start 142.216671 101.807836) (end 141.20706 101.807836) (width 0.1) (layer "F.Cu") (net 2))
 (segment (start 143.463413 102.093815) (end 151.802271 107.613185) (width 0.1) (layer "F.Cu") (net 2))
 (segment (start 151.664287 107.821657) (end 143.325429 102.302287) (width 0.1) (layer "F.Cu") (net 2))
 (segment (start 110.4 91.4) (end 110.4 101.314896) (width 0.1) (layer "F.Cu") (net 2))
 (segment (start 114.9 101.4) (end 114.9 91.4) (width 0.1) (layer "F.Cu") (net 2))
 (segment (start 112.15 101.4) (end 112.4 101.4) (width 0.1) (layer "F.Cu") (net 2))
 (segment (start 151.526303 108.030128) (end 151.664287 107.821657) (width 0.1) (layer "F.Cu") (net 2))
 (segment (start 113.65 101.4) (end 113.9 101.4) (width 0.1) (layer "F.Cu") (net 2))
 (segment (start 145.533177 98.966744) (end 145.671161 98.758272) (width 0.1) (layer "F.Cu") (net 2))
 (segment (start 112.4 101.4) (end 112.4 91.4) (width 0.1) (layer "F.Cu") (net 2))
 (segment (start 115.15706 103.207836) (end 116.80706 104.857836) (width 0.1) (layer "F.Cu") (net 2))
 (segment (start 142.395253 101.986418) (end 151.526303 108.030128) (width 0.1) (layer "F.Cu") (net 2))
 (segment (start 114.9 91.4) (end 115.15 91.4) (width 0.1) (layer "F.Cu") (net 2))
 (segment (start 151.940255 107.404714) (end 143.601397 101.885344) (width 0.1) (layer "F.Cu") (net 2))
 (segment (start 144.843255 100.009101) (end 153.182114 105.528471) (width 0.1) (layer "F.Cu") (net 2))
 (segment (start 145.119224 99.592158) (end 153.458082 105.111528) (width 0.1) (layer "F.Cu") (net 2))
 (segment (start 153.182114 105.528471) (end 153.320098 105.319999) (width 0.1) (layer "F.Cu") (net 2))
 (segment (start 111.65 91.4) (end 111.65 101.4) (width 0.1) (layer "F.Cu") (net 2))
 (segment (start 151.802271 107.613185) (end 151.940255 107.404714) (width 0.1) (layer "F.Cu") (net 2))
 (segment (start 112.65 101.4) (end 112.9 101.4) (width 0.1) (layer "F.Cu") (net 2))
 (segment (start 113.65 91.4) (end 113.65 101.4) (width 0.1) (layer "F.Cu") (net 2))
 (segment (start 154.010019 104.277642) (end 154.148003 104.069171) (width 0.1) (layer "F.Cu") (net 2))
 (segment (start 153.734051 104.694585) (end 153.872035 104.486113) (width 0.1) (layer "F.Cu") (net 2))
 (segment (start 144.98124 99.800629) (end 145.119224 99.592158) (width 0.1) (layer "F.Cu") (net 2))
 (segment (start 144.567287 100.426044) (end 152.906145 105.945414) (width 0.1) (layer "F.Cu") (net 2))
 (segment (start 153.320098 105.319999) (end 144.98124 99.800629) (width 0.1) (layer "F.Cu") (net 2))
 (segment (start 112.65 91.4) (end 112.65 101.4) (width 0.1) (layer "F.Cu") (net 2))
 (segment (start 153.596066 104.903056) (end 145.257208 99.383687) (width 0.1) (layer "F.Cu") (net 2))
 (segment (start 152.630177 106.362357) (end 152.768161 106.153885) (width 0.1) (layer "F.Cu") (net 2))
 (segment (start 142.395253 101.986418) (end 142.216671 101.807836) (width 0.1) (layer "F.Cu") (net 2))
 (segment (start 111.4 91.4) (end 111.65 91.4) (width 0.1) (layer "F.Cu") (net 2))
 (segment (start 152.07824 107.196242) (end 152.216224 106.987771) (width 0.1) (layer "F.Cu") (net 2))
 (segment (start 152.216224 106.987771) (end 143.877366 101.468401) (width 0.1) (layer "F.Cu") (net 2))
 (segment (start 111.65 101.4) (end 111.9 101.4) (width 0.1) (layer "F.Cu") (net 2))
 (segment (start 112.9 101.4) (end 112.9 91.4) (width 0.1) (layer "F.Cu") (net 2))
 (segment (start 143.739381 101.676873) (end 152.07824 107.196242) (width 0.1) (layer "F.Cu") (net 2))
 (segment (start 144.429303 100.634515) (end 144.567287 100.426044) (width 0.1) (layer "F.Cu") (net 2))
 (segment (start 152.906145 105.945414) (end 153.044129 105.736942) (width 0.1) (layer "F.Cu") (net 2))
 (segment (start 144.01535 101.25993) (end 152.354208 106.7793) (width 0.1) (layer "F.Cu") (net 2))
 (segment (start 112.9 91.4) (end 113.15 91.4) (width 0.1) (layer "F.Cu") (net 2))
 (segment (start 113.15 91.4) (end 113.15 101.4) (width 0.1) (layer "F.Cu") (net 2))
 (segment (start 114.4 101.4) (end 114.4 91.4) (width 0.1) (layer "F.Cu") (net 2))
 (segment (start 145.671161 98.758272) (end 154.010019 104.277642) (width 0.1) (layer "F.Cu") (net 2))
 (segment (start 110.65 91.4) (end 110.65 101.4) (width 0.1) (layer "F.Cu") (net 2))
 (segment (start 144.291318 100.842987) (end 152.630177 106.362357) (width 0.1) (layer "F.Cu") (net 2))
 (segment (start 111.15 91.4) (end 111.15 101.4) (width 0.1) (layer "F.Cu") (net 2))
 (segment (start 113.4 101.4) (end 113.4 91.4) (width 0.1) (layer "F.Cu") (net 2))
 (segment (start 112.15 91.4) (end 112.15 101.4) (width 0.1) (layer "F.Cu") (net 2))
 (segment (start 153.044129 105.736942) (end 144.705271 100.217572) (width 0.1) (layer "F.Cu") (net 2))
 (segment (start 110.65 101.4) (end 110.9 101.4) (width 0.1) (layer "F.Cu") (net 2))
 (segment (start 111.4 101.4) (end 111.4 91.4) (width 0.1) (layer "F.Cu") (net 2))
 (segment (start 114.65 91.4) (end 114.65 101.4) (width 0.1) (layer "F.Cu") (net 2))
 (segment (start 145.395192 99.175215) (end 153.734051 104.694585) (width 0.1) (layer "F.Cu") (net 2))
 (segment (start 152.492192 106.570828) (end 144.153334 101.051458) (width 0.1) (layer "F.Cu") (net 2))
 (segment (start 112.4 91.4) (end 112.65 91.4) (width 0.1) (layer "F.Cu") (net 2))
 (segment (start 113.4 91.4) (end 113.65 91.4) (width 0.1) (layer "F.Cu") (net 2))
 (segment (start 113.15 101.4) (end 113.4 101.4) (width 0.1) (layer "F.Cu") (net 2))
 (segment (start 115.15706 102.35706) (end 115.15706 103.207836) (width 0.1) (layer "F.Cu") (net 2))
 (segment (start 110.9 101.4) (end 110.9 91.4) (width 0.1) (layer "F.Cu") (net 2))
 (segment (start 145.016953 98.025461) (end 143.899328 96.907836) (width 0.1) (layer "F.Cu") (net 2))
 (segment (start 114.15 101.4) (end 114.4 101.4) (width 0.1) (layer "F.Cu") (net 2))
 (segment (start 145.257208 99.383687) (end 145.395192 99.175215) (width 0.1) (layer "F.Cu") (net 2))
 (segment (start 110.4 91.4) (end 110.65 91.4) (width 0.1) (layer "F.Cu") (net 2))
 (segment (start 143.601397 101.885344) (end 143.739381 101.676873) (width 0.1) (layer "F.Cu") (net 2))
 (segment (start 143.877366 101.468401) (end 144.01535 101.25993) (width 0.1) (layer "F.Cu") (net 2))
 (segment (start 113.9 101.4) (end 113.9 91.4) (width 0.1) (layer "F.Cu") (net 2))
 (segment (start 152.354208 106.7793) (end 152.492192 106.570828) (width 0.1) (layer "F.Cu") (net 2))
 (segment (start 143.899328 96.907836) (end 143.20706 96.907836) (width 0.1) (layer "F.Cu") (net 2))
 (via (at 138.25706 101.807836) (size 0.6) (drill 0.3) (layers "F.Cu" "B.Cu") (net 2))
 (via (at 116.80706 104.857836) (size 0.6) (drill 0.3) (layers "F.Cu" "B.Cu") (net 2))
 (segment (start 119.85706 101.807836) (end 116.80706 104.857836) (width 0.1) (layer "B.Cu") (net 2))
 (segment (start 116.80706 104.857836) (end 118.78706 106.837836) (width 0.1) (layer "B.Cu") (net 2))
 (segment (start 138.25706 101.807836) (end 119.85706 101.807836) (width 0.1) (layer "B.Cu") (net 2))
 (segment (start 118.78706 106.837836) (end 118.78706 107.907836) (width 0.1) (layer "B.Cu") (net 2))
 (segment (start 110.15706 106.457836) (end 124.95706 106.457836) (width 0.2) (layer "F.Cu") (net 4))
 (segment (start 124.95706 106.457836) (end 126.40706 107.907836) (width 0.2) (layer "F.Cu") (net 4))
 (segment (start 108.10706 104.407836) (end 110.15706 106.457836) (width 0.2) (layer "F.Cu") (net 4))
 (segment (start 107.90706 103.007836) (end 107.90706 104.207836) (width 0.2) (layer "F.Cu") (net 4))
 (segment (start 107.90706 104.207836) (end 108.10706 104.407836) (width 0.2) (layer "F.Cu") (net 4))
 (segment (start 141.20706 96.907836) (end 139.94706 96.907836) (width 0.2) (layer "F.Cu") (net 3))
 (segment (start 141.20706 96.907836) (end 142.60706 96.907836) (width 0.2) (layer "F.Cu") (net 3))
 (segment (start 139.94706 96.907836) (end 128.94706 107.907836) (width 0.2) (layer "F.Cu") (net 3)))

